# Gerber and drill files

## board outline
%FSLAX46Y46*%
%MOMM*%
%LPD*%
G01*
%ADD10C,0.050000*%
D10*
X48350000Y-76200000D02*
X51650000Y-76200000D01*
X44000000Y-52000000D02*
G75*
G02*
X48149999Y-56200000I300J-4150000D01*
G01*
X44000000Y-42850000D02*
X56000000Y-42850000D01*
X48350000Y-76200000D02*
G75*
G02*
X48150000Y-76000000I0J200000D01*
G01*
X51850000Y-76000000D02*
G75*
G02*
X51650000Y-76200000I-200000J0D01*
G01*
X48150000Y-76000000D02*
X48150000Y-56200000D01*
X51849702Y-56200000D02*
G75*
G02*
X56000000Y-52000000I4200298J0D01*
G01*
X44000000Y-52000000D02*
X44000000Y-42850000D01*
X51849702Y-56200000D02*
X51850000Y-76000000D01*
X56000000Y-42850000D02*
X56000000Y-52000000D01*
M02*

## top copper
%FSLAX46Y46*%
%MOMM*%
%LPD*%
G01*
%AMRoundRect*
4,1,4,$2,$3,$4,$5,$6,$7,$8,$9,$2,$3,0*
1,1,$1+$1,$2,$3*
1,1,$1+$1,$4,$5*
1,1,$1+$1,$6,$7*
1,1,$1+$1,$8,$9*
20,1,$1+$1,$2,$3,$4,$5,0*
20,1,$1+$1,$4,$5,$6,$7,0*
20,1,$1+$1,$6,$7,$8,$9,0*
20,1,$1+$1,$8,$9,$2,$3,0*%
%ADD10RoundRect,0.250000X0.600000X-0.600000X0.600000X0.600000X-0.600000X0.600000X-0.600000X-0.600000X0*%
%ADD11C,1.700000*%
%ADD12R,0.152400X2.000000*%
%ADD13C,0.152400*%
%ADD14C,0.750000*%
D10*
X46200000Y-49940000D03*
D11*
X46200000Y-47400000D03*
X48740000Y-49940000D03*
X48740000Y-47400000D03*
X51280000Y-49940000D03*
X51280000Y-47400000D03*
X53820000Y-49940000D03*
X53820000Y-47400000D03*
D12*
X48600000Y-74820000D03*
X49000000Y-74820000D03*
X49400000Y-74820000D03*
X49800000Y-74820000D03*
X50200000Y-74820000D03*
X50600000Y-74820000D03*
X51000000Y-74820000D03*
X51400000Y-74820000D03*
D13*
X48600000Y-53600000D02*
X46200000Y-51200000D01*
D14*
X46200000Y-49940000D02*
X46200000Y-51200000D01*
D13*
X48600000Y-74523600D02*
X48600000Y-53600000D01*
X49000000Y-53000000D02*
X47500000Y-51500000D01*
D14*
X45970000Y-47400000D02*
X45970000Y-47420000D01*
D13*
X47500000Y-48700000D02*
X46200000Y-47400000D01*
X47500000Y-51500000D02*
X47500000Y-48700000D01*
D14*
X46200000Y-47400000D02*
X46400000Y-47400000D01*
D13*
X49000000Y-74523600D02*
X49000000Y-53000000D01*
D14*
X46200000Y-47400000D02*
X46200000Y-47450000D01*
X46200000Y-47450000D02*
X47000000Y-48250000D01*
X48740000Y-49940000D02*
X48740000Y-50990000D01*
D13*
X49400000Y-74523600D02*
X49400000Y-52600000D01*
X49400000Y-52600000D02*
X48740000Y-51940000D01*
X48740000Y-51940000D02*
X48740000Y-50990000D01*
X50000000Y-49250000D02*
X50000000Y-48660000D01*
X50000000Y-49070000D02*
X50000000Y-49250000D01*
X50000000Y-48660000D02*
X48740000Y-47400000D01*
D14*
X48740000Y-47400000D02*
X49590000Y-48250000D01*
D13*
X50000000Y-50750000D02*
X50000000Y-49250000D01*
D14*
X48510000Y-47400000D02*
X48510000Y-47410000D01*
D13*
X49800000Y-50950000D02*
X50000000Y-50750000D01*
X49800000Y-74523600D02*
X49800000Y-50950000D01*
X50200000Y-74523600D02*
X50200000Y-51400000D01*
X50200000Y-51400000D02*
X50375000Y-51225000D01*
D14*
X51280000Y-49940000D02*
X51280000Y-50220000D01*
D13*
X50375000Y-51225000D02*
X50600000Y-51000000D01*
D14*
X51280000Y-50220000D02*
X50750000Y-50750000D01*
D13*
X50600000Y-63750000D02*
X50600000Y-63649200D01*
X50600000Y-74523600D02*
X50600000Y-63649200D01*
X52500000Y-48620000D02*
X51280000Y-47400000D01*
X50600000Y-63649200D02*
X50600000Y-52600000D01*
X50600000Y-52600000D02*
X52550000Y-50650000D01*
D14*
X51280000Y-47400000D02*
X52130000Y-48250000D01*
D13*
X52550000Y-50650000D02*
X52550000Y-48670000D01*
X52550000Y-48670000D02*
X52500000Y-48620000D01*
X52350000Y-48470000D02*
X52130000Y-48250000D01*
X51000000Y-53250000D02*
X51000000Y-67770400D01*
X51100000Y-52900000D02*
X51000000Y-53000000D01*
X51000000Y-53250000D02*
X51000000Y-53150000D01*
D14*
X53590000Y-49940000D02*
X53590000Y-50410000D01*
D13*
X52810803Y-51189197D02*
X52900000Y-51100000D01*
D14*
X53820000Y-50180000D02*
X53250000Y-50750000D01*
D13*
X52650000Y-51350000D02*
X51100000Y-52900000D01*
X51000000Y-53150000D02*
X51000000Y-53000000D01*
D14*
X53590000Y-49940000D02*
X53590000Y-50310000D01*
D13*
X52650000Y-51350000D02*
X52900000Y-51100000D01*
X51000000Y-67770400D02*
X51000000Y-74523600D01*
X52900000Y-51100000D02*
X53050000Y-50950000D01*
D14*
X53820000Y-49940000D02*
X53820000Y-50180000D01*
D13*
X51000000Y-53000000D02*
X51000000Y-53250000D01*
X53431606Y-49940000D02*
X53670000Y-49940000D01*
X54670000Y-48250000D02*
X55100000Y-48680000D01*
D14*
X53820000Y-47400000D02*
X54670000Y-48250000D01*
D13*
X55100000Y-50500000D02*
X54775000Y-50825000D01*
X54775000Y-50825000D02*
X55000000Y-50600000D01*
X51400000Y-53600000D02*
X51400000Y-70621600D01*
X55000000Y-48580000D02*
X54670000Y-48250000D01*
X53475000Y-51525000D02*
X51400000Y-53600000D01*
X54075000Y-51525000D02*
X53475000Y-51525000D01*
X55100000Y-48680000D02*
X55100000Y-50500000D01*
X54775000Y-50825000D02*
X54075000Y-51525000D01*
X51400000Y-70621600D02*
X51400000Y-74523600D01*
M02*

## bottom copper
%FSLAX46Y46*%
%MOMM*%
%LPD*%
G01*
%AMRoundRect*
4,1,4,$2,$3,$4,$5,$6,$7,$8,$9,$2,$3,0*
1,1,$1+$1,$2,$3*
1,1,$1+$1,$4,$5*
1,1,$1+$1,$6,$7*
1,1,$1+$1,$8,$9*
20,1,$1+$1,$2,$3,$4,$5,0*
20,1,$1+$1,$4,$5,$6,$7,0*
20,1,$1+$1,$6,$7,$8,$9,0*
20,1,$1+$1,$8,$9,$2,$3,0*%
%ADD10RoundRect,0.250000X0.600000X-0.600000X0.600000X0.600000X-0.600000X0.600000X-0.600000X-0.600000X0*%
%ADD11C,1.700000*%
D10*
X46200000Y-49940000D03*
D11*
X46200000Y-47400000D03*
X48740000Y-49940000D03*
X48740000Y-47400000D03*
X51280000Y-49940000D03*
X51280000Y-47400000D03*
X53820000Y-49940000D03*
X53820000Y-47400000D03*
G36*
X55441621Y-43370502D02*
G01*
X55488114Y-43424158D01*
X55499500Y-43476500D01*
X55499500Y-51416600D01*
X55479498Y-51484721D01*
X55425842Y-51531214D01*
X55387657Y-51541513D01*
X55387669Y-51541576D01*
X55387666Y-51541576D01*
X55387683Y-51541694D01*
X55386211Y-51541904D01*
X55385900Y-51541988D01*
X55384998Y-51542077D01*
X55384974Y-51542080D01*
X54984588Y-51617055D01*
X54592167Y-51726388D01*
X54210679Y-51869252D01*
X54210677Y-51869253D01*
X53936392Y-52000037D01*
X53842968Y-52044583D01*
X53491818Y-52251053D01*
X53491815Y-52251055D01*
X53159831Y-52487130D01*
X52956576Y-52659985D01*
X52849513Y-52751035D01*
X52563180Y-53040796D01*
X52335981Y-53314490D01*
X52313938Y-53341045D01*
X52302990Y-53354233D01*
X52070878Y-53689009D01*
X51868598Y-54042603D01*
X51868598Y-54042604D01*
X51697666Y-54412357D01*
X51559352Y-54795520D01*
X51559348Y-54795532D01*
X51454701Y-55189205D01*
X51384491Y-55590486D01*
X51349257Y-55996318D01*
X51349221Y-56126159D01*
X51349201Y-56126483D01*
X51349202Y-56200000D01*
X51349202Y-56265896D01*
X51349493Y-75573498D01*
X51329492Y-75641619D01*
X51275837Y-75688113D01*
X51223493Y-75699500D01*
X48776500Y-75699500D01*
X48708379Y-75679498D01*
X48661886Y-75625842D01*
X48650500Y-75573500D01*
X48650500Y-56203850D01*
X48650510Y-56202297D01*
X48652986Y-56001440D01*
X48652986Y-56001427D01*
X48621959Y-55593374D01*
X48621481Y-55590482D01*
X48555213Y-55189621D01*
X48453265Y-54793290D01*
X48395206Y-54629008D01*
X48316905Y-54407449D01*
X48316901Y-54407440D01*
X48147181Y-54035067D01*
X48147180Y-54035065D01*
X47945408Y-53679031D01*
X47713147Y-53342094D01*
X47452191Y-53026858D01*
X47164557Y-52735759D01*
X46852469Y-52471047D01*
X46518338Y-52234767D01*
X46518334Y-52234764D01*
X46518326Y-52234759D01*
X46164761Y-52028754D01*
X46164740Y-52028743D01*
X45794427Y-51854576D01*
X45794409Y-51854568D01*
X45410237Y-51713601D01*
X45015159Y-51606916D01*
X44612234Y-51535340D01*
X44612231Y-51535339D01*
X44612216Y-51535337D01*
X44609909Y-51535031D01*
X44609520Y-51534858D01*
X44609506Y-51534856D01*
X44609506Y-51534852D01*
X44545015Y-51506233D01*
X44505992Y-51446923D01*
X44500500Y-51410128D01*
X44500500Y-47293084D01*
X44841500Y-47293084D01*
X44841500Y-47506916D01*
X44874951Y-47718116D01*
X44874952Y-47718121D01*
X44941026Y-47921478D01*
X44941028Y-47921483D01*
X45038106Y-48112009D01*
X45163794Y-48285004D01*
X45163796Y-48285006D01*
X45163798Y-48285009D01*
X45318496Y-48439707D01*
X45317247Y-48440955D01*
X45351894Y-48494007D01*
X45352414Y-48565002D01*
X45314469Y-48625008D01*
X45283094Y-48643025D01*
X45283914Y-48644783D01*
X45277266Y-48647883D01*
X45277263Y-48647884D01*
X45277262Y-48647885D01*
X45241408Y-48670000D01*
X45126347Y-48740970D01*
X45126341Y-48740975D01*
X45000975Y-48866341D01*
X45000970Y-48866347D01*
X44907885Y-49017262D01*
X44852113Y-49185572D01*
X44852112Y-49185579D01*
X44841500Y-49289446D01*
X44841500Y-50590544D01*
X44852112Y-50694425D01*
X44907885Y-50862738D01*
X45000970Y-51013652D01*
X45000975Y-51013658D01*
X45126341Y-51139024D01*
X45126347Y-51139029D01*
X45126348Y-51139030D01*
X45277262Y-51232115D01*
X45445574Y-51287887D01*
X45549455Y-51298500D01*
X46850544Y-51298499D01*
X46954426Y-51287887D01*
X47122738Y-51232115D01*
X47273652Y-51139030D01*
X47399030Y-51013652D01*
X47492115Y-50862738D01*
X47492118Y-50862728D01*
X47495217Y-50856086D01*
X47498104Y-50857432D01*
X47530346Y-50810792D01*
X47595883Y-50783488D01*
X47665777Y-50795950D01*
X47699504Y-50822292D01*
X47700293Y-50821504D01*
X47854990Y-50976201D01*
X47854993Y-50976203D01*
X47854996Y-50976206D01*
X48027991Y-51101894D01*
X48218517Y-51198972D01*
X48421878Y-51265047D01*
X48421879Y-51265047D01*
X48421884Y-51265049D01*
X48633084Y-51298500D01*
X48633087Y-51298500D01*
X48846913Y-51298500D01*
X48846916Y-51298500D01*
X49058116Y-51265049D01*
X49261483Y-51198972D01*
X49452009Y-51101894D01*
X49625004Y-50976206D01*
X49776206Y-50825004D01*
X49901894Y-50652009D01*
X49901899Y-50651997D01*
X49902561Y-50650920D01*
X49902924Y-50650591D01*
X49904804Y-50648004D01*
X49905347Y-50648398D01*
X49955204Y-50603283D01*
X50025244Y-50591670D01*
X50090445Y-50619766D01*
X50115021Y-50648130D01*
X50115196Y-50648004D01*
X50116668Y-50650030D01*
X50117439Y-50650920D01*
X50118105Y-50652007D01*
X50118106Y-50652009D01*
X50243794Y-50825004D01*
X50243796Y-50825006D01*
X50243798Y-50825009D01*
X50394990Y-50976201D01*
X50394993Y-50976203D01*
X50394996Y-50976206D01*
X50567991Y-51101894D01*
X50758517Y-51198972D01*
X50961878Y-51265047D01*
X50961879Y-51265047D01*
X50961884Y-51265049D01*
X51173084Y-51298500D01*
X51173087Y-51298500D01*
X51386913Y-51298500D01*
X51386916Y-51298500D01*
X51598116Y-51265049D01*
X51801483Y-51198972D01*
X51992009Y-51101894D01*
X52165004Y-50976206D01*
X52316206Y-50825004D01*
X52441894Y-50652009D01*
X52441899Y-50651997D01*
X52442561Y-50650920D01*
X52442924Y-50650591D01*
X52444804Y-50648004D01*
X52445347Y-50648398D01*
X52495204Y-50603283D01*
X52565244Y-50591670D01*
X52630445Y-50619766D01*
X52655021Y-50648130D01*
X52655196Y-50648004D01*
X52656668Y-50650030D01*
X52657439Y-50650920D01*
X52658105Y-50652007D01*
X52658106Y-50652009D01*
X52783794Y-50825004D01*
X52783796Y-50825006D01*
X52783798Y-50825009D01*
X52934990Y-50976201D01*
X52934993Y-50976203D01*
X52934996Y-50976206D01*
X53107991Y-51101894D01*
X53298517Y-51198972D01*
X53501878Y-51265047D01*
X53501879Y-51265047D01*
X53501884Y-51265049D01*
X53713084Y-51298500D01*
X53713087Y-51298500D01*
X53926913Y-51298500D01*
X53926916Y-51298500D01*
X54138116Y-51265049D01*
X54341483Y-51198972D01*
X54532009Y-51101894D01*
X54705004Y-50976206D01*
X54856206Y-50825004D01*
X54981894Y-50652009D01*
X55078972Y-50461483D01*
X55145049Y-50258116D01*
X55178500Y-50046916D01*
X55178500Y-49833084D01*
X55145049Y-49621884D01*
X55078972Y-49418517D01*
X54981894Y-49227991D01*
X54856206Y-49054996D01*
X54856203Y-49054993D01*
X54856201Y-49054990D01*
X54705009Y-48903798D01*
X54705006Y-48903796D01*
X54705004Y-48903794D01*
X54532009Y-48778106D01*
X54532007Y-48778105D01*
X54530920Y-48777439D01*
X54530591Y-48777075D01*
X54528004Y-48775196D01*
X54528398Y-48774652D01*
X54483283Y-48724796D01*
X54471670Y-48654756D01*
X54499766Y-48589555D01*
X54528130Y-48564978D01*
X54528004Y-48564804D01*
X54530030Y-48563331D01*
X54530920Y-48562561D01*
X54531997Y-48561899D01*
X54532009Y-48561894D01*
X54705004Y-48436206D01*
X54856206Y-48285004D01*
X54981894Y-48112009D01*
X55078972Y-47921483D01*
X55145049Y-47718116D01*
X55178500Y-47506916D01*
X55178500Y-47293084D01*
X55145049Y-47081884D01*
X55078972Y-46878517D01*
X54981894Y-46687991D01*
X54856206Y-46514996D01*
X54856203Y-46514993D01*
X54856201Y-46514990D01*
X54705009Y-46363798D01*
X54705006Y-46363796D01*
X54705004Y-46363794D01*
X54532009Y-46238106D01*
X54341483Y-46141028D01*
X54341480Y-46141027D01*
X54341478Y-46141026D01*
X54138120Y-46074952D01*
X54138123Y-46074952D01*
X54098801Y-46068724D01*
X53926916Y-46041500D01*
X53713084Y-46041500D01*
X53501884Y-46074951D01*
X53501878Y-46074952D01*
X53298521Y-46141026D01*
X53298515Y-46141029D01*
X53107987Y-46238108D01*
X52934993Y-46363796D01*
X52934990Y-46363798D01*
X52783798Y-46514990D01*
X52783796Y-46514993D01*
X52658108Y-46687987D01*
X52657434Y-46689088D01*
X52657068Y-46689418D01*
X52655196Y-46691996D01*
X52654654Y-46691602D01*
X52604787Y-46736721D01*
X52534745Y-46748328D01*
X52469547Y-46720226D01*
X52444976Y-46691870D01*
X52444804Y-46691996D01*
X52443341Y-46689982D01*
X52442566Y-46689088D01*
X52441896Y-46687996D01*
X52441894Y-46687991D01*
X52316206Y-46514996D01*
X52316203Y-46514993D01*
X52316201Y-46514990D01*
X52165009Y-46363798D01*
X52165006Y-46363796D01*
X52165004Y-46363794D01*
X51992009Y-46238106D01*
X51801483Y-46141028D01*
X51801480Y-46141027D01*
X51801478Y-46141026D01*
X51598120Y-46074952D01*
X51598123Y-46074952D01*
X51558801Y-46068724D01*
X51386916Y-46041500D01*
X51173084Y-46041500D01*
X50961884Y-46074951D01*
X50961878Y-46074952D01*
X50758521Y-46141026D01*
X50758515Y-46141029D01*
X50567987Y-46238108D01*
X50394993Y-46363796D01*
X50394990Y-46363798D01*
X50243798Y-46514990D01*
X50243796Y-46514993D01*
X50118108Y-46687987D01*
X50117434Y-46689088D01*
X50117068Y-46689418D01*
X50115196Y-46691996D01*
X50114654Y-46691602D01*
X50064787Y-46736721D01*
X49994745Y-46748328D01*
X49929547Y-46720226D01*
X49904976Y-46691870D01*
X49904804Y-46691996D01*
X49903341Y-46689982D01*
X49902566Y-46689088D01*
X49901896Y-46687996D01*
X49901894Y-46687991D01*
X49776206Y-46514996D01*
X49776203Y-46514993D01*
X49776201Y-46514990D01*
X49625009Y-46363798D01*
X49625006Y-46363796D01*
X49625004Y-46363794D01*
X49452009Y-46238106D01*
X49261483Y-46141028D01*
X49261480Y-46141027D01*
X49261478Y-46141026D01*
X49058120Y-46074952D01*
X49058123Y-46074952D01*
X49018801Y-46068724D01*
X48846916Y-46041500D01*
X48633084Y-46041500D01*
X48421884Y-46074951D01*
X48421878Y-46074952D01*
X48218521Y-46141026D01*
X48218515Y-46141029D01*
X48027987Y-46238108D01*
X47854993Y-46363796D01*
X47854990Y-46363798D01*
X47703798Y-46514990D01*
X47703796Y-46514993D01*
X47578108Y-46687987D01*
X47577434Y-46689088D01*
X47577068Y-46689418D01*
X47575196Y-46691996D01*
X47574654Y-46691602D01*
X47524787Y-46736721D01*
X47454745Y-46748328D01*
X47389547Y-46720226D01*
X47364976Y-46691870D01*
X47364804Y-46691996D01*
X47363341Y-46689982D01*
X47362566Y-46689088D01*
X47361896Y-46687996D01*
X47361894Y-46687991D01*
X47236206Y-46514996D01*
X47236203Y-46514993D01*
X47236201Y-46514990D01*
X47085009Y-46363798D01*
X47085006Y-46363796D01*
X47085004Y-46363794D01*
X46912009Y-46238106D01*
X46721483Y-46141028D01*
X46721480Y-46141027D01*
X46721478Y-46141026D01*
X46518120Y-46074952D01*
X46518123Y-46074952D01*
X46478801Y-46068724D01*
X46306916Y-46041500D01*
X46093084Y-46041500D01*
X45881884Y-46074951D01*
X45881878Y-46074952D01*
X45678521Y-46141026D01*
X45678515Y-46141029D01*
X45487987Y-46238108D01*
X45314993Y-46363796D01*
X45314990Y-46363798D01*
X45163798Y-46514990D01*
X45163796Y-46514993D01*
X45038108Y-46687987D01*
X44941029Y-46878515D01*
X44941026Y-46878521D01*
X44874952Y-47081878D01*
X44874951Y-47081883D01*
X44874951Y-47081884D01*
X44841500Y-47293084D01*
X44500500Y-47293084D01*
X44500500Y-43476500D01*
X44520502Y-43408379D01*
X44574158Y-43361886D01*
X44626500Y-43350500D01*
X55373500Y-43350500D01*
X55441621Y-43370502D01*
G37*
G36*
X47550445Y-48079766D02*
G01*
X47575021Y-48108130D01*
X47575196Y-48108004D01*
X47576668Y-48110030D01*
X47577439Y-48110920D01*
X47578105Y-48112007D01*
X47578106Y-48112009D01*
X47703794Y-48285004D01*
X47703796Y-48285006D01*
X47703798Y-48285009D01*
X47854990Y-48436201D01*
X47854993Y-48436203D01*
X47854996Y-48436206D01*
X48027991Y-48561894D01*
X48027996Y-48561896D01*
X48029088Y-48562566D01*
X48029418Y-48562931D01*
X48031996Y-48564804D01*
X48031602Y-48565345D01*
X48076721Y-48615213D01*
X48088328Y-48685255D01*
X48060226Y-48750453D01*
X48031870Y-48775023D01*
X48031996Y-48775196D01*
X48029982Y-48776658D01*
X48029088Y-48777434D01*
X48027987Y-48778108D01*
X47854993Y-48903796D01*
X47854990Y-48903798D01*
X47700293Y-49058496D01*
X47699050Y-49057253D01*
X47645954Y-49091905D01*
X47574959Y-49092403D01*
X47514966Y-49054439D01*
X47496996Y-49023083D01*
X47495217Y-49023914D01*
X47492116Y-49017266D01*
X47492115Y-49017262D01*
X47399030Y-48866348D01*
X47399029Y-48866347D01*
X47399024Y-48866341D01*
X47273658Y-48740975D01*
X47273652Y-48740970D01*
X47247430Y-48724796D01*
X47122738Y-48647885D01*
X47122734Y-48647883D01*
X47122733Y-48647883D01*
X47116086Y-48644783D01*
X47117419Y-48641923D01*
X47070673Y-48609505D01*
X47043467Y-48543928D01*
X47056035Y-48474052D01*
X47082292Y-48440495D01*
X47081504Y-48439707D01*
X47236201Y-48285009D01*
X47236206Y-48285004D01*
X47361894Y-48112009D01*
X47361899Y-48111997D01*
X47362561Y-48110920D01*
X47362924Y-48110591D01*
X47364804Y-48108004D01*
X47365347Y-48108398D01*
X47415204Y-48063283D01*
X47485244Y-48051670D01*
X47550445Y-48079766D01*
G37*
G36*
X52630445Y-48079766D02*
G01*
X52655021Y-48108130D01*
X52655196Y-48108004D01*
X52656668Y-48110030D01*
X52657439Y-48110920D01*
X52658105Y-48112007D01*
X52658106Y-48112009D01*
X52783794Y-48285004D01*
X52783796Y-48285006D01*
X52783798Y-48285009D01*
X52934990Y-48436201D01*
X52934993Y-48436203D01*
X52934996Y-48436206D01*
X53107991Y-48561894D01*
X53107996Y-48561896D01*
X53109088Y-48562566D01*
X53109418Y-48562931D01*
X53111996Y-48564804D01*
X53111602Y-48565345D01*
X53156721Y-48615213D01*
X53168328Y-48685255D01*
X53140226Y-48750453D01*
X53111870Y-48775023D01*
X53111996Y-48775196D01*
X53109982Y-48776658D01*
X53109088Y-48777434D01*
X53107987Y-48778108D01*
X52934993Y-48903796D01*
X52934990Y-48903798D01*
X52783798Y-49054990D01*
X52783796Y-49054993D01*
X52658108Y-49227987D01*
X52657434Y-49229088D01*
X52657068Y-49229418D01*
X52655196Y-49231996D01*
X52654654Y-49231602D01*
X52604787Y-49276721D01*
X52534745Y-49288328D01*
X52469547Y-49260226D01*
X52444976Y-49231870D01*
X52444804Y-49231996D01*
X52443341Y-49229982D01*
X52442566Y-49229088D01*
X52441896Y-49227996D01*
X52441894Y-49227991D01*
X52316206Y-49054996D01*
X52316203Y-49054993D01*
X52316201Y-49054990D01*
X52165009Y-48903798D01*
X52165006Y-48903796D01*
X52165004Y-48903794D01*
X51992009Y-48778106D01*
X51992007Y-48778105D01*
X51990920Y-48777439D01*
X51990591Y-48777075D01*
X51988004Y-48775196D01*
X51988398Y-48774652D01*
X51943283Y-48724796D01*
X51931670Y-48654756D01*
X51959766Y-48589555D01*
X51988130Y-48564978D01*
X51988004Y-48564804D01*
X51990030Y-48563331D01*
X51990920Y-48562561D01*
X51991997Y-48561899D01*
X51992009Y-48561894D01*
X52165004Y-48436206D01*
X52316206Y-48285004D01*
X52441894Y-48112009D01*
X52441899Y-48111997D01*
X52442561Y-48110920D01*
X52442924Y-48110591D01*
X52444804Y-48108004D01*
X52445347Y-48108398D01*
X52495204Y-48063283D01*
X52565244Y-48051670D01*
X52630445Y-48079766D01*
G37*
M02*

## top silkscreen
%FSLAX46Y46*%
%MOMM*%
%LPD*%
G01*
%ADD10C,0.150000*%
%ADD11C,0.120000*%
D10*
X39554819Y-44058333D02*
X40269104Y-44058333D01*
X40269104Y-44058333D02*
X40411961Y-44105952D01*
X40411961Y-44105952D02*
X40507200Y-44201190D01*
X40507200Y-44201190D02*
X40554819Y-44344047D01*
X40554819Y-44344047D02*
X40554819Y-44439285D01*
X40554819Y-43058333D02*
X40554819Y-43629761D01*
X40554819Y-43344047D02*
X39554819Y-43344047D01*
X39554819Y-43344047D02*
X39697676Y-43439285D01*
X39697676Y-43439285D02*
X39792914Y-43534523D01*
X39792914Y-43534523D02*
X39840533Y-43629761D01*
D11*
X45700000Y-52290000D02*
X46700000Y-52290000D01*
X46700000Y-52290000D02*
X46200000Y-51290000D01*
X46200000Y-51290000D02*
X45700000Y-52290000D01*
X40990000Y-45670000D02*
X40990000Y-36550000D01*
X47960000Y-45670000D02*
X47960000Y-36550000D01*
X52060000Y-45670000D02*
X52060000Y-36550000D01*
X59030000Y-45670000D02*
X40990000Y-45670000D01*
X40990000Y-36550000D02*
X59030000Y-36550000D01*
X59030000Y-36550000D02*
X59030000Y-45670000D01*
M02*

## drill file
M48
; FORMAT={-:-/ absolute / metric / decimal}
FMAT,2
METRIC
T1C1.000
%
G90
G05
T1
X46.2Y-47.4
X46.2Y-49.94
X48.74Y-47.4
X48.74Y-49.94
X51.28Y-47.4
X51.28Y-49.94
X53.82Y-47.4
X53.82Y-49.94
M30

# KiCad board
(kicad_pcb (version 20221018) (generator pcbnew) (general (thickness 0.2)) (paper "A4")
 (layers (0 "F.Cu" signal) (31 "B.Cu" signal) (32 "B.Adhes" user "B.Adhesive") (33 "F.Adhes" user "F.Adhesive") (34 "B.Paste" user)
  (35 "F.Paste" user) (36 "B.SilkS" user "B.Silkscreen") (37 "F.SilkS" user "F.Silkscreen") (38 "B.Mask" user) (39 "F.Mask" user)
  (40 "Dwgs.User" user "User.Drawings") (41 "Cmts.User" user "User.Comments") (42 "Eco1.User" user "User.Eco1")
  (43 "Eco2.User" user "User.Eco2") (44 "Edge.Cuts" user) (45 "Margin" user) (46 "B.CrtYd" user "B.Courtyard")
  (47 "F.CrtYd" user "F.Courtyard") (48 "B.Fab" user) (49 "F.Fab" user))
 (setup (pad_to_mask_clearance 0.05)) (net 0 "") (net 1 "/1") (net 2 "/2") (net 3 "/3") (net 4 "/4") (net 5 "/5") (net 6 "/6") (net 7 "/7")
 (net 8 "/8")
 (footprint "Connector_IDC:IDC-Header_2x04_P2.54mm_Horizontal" (layer "F.Cu") (at 46.2 49.94 90)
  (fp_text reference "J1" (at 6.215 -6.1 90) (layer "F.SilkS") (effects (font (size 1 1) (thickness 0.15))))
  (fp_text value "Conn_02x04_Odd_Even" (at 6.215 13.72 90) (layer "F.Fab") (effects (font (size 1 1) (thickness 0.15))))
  (fp_line (start -2.35 -0.5) (end -2.35 0.5) (stroke (width 0.12) (type solid)) (layer "F.SilkS"))
  (fp_line (start -2.35 0.5) (end -1.35 0) (stroke (width 0.12) (type solid)) (layer "F.SilkS"))
  (fp_line (start -1.35 0) (end -2.35 -0.5) (stroke (width 0.12) (type solid)) (layer "F.SilkS"))
  (fp_line (start 4.27 -5.21) (end 13.39 -5.21) (stroke (width 0.12) (type solid)) (layer "F.SilkS"))
  (fp_line (start 4.27 1.76) (end 13.39 1.76) (stroke (width 0.12) (type solid)) (layer "F.SilkS"))
  (fp_line (start 4.27 5.86) (end 13.39 5.86) (stroke (width 0.12) (type solid)) (layer "F.SilkS"))
  (fp_line (start 4.27 12.83) (end 4.27 -5.21) (stroke (width 0.12) (type solid)) (layer "F.SilkS"))
  (fp_line (start 13.39 -5.21) (end 13.39 12.83) (stroke (width 0.12) (type solid)) (layer "F.SilkS"))
  (fp_line (start 13.39 12.83) (end 4.27 12.83) (stroke (width 0.12) (type solid)) (layer "F.SilkS"))
  (pad "1" thru_hole roundrect (at 0 0 90) (size 1.7 1.7) (drill 1) (layers "*.Cu" "*.Mask") (roundrect_rratio 0.1470588235) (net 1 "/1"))
  (pad "2" thru_hole circle (at 2.54 0 90) (size 1.7 1.7) (drill 1) (layers "*.Cu" "*.Mask") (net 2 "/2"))
  (pad "3" thru_hole circle (at 0 2.54 90) (size 1.7 1.7) (drill 1) (layers "*.Cu" "*.Mask") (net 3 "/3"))
  (pad "4" thru_hole circle (at 2.54 2.54 90) (size 1.7 1.7) (drill 1) (layers "*.Cu" "*.Mask") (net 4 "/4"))
  (pad "5" thru_hole circle (at 0 5.08 90) (size 1.7 1.7) (drill 1) (layers "*.Cu" "*.Mask") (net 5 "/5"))
  (pad "6" thru_hole circle (at 2.54 5.08 90) (size 1.7 1.7) (drill 1) (layers "*.Cu" "*.Mask") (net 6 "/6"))
  (pad "7" thru_hole circle (at 0 7.62 90) (size 1.7 1.7) (drill 1) (layers "*.Cu" "*.Mask") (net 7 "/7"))
  (pad "8" thru_hole circle (at 2.54 7.62 90) (size 1.7 1.7) (drill 1) (layers "*.Cu" "*.Mask") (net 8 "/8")))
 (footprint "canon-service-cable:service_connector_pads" (layer "F.Cu") (at 48.25 74.57)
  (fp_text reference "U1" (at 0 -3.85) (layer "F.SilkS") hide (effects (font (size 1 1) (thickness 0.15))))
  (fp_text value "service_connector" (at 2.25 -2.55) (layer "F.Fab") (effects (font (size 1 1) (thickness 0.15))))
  (pad "1" smd rect (at 0.35 0.25) (size 0.1524 2) (layers "F.Cu" "F.Paste" "F.Mask") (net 1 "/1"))
  (pad "2" smd rect (at 0.75 0.25) (size 0.1524 2) (layers "F.Cu" "F.Paste" "F.Mask") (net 2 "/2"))
  (pad "3" smd rect (at 1.15 0.25) (size 0.1524 2) (layers "F.Cu" "F.Paste" "F.Mask") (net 3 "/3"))
  (pad "4" smd rect (at 1.55 0.25) (size 0.1524 2) (layers "F.Cu" "F.Paste" "F.Mask") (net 4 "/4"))
  (pad "5" smd rect (at 1.95 0.25) (size 0.1524 2) (layers "F.Cu" "F.Paste" "F.Mask") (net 5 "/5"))
  (pad "6" smd rect (at 2.35 0.25) (size 0.1524 2) (layers "F.Cu" "F.Paste" "F.Mask") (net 6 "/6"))
  (pad "7" smd rect (at 2.75 0.25) (size 0.1524 2) (layers "F.Cu" "F.Paste" "F.Mask") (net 7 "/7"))
  (pad "8" smd rect (at 3.15 0.25) (size 0.1524 2) (layers "F.Cu" "F.Paste" "F.Mask") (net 8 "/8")))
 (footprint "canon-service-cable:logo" (layer "B.Cu") (at 48.11 54 180)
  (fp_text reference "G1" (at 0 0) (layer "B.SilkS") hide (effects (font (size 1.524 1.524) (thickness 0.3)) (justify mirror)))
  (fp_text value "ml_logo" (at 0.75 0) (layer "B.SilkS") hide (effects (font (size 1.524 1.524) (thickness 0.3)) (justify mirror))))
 (gr_line (start 48.35 76.2) (end 51.65 76.2) (stroke (width 0.05) (type solid)) (layer "Edge.Cuts"))
 (gr_arc (start 44 52) (mid 46.952314 53.23313) (end 48.15 56.2) (stroke (width 0.05) (type solid)) (layer "Edge.Cuts"))
 (gr_line (start 44 42.85) (end 56 42.85) (stroke (width 0.05) (type solid)) (layer "Edge.Cuts"))
 (gr_arc (start 48.35 76.2) (mid 48.208579 76.141421) (end 48.15 76) (stroke (width 0.05) (type solid)) (layer "Edge.Cuts"))
 (gr_arc (start 51.85 76) (mid 51.791421 76.141421) (end 51.65 76.2) (stroke (width 0.05) (type solid)) (layer "Edge.Cuts"))
 (gr_line (start 48.15 76) (end 48.15 56.2) (stroke (width 0.05) (type solid)) (layer "Edge.Cuts"))
 (gr_arc (start 51.849702 56.2) (mid 53.062315 53.247671) (end 56 52) (stroke (width 0.05) (type solid)) (layer "Edge.Cuts"))
 (gr_line (start 44 52) (end 44 42.85) (stroke (width 0.05) (type solid)) (layer "Edge.Cuts"))
 (gr_line (start 51.849702 56.2) (end 51.85 76) (stroke (width 0.05) (type solid)) (layer "Edge.Cuts"))
 (gr_line (start 56 42.85) (end 56 52) (stroke (width 0.05) (type solid)) (layer "Edge.Cuts"))
 (segment (start 48.6 53.6) (end 46.2 51.2) (width 0.1524) (layer "F.Cu") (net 1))
 (segment (start 46.2 49.94) (end 46.2 51.2) (width 0.75) (layer "F.Cu") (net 1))
 (segment (start 48.6 74.5236) (end 48.6 53.6) (width 0.1524) (layer "F.Cu") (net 1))
 (segment (start 49 53) (end 47.5 51.5) (width 0.1524) (layer "F.Cu") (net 2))
 (segment (start 45.97 47.4) (end 45.97 47.42) (width 0.75) (layer "F.Cu") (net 2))
 (segment (start 47.5 48.7) (end 46.2 47.4) (width 0.1524) (layer "F.Cu") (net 2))
 (segment (start 47.5 51.5) (end 47.5 48.7) (width 0.1524) (layer "F.Cu") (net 2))
 (segment (start 46.2 47.4) (end 46.4 47.4) (width 0.75) (layer "F.Cu") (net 2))
 (segment (start 49 74.5236) (end 49 53) (width 0.1524) (layer "F.Cu") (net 2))
 (segment (start 46.2 47.4) (end 46.2 47.45) (width 0.75) (layer "F.Cu") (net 2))
 (segment (start 46.2 47.45) (end 47 48.25) (width 0.75) (layer "F.Cu") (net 2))
 (segment (start 48.74 49.94) (end 48.74 50.99) (width 0.75) (layer "F.Cu") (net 3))
 (segment (start 49.4 74.5236) (end 49.4 52.6) (width 0.1524) (layer "F.Cu") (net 3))
 (segment (start 49.4 52.6) (end 48.74 51.94) (width 0.1524) (layer "F.Cu") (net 3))
 (segment (start 48.74 51.94) (end 48.74 50.99) (width 0.1524) (layer "F.Cu") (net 3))
 (segment (start 50 49.25) (end 50 48.66) (width 0.1524) (layer "F.Cu") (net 4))
 (segment (start 50 49.07) (end 50 49.25) (width 0.1524) (layer "F.Cu") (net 4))
 (segment (start 50 48.66) (end 48.74 47.4) (width 0.1524) (layer "F.Cu") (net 4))
 (segment (start 48.74 47.4) (end 49.59 48.25) (width 0.75) (layer "F.Cu") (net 4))
 (segment (start 50 50.75) (end 50 49.25) (width 0.1524) (layer "F.Cu") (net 4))
 (segment (start 48.51 47.4) (end 48.51 47.41) (width 0.75) (layer "F.Cu") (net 4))
 (segment (start 49.8 50.95) (end 50 50.75) (width 0.1524) (layer "F.Cu") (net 4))
 (segment (start 49.8 74.5236) (end 49.8 50.95) (width 0.1524) (layer "F.Cu") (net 4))
 (segment (start 50.2 74.5236) (end 50.2 51.4) (width 0.1524) (layer "F.Cu") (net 5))
 (segment (start 50.2 51.4) (end 50.375 51.225) (width 0.1524) (layer "F.Cu") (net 5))
 (segment (start 51.28 49.94) (end 51.28 50.22) (width 0.75) (layer "F.Cu") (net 5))
 (segment (start 50.375 51.225) (end 50.6 51) (width 0.1524) (layer "F.Cu") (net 5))
 (segment (start 51.28 50.22) (end 50.75 50.75) (width 0.75) (layer "F.Cu") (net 5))
 (segment (start 50.6 63.75) (end 50.6 63.6492) (width 0.1524) (layer "F.Cu") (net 6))
 (segment (start 50.6 74.5236) (end 50.6 63.6492) (width 0.1524) (layer "F.Cu") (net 6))
 (segment (start 52.5 48.62) (end 51.28 47.4) (width 0.1524) (layer "F.Cu") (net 6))
 (segment (start 50.6 63.6492) (end 50.6 52.6) (width 0.1524) (layer "F.Cu") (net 6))
 (segment (start 50.6 52.6) (end 52.55 50.65) (width 0.1524) (layer "F.Cu") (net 6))
 (segment (start 51.28 47.4) (end 52.13 48.25) (width 0.75) (layer "F.Cu") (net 6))
 (segment (start 52.55 50.65) (end 52.55 48.67) (width 0.1524) (layer "F.Cu") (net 6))
 (segment (start 52.55 48.67) (end 52.5 48.62) (width 0.1524) (layer "F.Cu") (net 6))
 (segment (start 52.35 48.47) (end 52.13 48.25) (width 0.1524) (layer "F.Cu") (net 6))
 (segment (start 51 53.25) (end 51 67.7704) (width 0.1524) (layer "F.Cu") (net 7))
 (segment (start 51.1 52.9) (end 51 53) (width 0.1524) (layer "F.Cu") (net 7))
 (segment (start 51 53.25) (end 51 53.15) (width 0.1524) (layer "F.Cu") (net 7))
 (segment (start 53.59 49.94) (end 53.59 50.41) (width 0.75) (layer "F.Cu") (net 7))
 (segment (start 52.810803 51.189197) (end 52.9 51.1) (width 0.1524) (layer "F.Cu") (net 7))
 (segment (start 53.82 50.18) (end 53.25 50.75) (width 0.75) (layer "F.Cu") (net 7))
 (segment (start 52.65 51.35) (end 51.1 52.9) (width 0.1524) (layer "F.Cu") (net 7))
 (segment (start 51 53.15) (end 51 53) (width 0.1524) (layer "F.Cu") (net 7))
 (segment (start 53.59 49.94) (end 53.59 50.31) (width 0.75) (layer "F.Cu") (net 7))
 (segment (start 52.65 51.35) (end 52.9 51.1) (width 0.1524) (layer "F.Cu") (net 7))
 (segment (start 51 67.7704) (end 51 74.5236) (width 0.1524) (layer "F.Cu") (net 7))
 (segment (start 52.9 51.1) (end 53.05 50.95) (width 0.1524) (layer "F.Cu") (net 7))
 (segment (start 53.82 49.94) (end 53.82 50.18) (width 0.75) (layer "F.Cu") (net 7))
 (segment (start 51 53) (end 51 53.25) (width 0.1524) (layer "F.Cu") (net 7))
 (segment (start 53.431606 49.94) (end 53.67 49.94) (width 0.1524) (layer "F.Cu") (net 7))
 (segment (start 54.67 48.25) (end 55.1 48.68) (width 0.1524) (layer "F.Cu") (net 8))
 (segment (start 53.82 47.4) (end 54.67 48.25) (width 0.75) (layer "F.Cu") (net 8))
 (segment (start 55.1 50.5) (end 54.775 50.825) (width 0.1524) (layer "F.Cu") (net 8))
 (segment (start 54.775 50.825) (end 55 50.6) (width 0.1524) (layer "F.Cu") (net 8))
 (segment (start 51.4 53.6) (end 51.4 70.6216) (width 0.1524) (layer "F.Cu") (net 8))
 (segment (start 55 48.58) (end 54.67 48.25) (width 0.1524) (layer "F.Cu") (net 8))
 (segment (start 53.475 51.525) (end 51.4 53.6) (width 0.1524) (layer "F.Cu") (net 8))
 (segment (start 54.075 51.525) (end 53.475 51.525) (width 0.1524) (layer "F.Cu") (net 8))
 (segment (start 55.1 48.68) (end 55.1 50.5) (width 0.1524) (layer "F.Cu") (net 8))
 (segment (start 54.775 50.825) (end 54.075 51.525) (width 0.1524) (layer "F.Cu") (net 8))
 (segment (start 51.4 70.6216) (end 51.4 74.5236) (width 0.1524) (layer "F.Cu") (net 8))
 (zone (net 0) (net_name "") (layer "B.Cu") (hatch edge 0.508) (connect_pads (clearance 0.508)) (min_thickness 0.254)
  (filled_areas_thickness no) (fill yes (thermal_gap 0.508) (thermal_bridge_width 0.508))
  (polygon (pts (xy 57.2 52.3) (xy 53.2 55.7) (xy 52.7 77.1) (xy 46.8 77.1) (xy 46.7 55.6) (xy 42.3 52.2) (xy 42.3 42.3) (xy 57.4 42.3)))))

